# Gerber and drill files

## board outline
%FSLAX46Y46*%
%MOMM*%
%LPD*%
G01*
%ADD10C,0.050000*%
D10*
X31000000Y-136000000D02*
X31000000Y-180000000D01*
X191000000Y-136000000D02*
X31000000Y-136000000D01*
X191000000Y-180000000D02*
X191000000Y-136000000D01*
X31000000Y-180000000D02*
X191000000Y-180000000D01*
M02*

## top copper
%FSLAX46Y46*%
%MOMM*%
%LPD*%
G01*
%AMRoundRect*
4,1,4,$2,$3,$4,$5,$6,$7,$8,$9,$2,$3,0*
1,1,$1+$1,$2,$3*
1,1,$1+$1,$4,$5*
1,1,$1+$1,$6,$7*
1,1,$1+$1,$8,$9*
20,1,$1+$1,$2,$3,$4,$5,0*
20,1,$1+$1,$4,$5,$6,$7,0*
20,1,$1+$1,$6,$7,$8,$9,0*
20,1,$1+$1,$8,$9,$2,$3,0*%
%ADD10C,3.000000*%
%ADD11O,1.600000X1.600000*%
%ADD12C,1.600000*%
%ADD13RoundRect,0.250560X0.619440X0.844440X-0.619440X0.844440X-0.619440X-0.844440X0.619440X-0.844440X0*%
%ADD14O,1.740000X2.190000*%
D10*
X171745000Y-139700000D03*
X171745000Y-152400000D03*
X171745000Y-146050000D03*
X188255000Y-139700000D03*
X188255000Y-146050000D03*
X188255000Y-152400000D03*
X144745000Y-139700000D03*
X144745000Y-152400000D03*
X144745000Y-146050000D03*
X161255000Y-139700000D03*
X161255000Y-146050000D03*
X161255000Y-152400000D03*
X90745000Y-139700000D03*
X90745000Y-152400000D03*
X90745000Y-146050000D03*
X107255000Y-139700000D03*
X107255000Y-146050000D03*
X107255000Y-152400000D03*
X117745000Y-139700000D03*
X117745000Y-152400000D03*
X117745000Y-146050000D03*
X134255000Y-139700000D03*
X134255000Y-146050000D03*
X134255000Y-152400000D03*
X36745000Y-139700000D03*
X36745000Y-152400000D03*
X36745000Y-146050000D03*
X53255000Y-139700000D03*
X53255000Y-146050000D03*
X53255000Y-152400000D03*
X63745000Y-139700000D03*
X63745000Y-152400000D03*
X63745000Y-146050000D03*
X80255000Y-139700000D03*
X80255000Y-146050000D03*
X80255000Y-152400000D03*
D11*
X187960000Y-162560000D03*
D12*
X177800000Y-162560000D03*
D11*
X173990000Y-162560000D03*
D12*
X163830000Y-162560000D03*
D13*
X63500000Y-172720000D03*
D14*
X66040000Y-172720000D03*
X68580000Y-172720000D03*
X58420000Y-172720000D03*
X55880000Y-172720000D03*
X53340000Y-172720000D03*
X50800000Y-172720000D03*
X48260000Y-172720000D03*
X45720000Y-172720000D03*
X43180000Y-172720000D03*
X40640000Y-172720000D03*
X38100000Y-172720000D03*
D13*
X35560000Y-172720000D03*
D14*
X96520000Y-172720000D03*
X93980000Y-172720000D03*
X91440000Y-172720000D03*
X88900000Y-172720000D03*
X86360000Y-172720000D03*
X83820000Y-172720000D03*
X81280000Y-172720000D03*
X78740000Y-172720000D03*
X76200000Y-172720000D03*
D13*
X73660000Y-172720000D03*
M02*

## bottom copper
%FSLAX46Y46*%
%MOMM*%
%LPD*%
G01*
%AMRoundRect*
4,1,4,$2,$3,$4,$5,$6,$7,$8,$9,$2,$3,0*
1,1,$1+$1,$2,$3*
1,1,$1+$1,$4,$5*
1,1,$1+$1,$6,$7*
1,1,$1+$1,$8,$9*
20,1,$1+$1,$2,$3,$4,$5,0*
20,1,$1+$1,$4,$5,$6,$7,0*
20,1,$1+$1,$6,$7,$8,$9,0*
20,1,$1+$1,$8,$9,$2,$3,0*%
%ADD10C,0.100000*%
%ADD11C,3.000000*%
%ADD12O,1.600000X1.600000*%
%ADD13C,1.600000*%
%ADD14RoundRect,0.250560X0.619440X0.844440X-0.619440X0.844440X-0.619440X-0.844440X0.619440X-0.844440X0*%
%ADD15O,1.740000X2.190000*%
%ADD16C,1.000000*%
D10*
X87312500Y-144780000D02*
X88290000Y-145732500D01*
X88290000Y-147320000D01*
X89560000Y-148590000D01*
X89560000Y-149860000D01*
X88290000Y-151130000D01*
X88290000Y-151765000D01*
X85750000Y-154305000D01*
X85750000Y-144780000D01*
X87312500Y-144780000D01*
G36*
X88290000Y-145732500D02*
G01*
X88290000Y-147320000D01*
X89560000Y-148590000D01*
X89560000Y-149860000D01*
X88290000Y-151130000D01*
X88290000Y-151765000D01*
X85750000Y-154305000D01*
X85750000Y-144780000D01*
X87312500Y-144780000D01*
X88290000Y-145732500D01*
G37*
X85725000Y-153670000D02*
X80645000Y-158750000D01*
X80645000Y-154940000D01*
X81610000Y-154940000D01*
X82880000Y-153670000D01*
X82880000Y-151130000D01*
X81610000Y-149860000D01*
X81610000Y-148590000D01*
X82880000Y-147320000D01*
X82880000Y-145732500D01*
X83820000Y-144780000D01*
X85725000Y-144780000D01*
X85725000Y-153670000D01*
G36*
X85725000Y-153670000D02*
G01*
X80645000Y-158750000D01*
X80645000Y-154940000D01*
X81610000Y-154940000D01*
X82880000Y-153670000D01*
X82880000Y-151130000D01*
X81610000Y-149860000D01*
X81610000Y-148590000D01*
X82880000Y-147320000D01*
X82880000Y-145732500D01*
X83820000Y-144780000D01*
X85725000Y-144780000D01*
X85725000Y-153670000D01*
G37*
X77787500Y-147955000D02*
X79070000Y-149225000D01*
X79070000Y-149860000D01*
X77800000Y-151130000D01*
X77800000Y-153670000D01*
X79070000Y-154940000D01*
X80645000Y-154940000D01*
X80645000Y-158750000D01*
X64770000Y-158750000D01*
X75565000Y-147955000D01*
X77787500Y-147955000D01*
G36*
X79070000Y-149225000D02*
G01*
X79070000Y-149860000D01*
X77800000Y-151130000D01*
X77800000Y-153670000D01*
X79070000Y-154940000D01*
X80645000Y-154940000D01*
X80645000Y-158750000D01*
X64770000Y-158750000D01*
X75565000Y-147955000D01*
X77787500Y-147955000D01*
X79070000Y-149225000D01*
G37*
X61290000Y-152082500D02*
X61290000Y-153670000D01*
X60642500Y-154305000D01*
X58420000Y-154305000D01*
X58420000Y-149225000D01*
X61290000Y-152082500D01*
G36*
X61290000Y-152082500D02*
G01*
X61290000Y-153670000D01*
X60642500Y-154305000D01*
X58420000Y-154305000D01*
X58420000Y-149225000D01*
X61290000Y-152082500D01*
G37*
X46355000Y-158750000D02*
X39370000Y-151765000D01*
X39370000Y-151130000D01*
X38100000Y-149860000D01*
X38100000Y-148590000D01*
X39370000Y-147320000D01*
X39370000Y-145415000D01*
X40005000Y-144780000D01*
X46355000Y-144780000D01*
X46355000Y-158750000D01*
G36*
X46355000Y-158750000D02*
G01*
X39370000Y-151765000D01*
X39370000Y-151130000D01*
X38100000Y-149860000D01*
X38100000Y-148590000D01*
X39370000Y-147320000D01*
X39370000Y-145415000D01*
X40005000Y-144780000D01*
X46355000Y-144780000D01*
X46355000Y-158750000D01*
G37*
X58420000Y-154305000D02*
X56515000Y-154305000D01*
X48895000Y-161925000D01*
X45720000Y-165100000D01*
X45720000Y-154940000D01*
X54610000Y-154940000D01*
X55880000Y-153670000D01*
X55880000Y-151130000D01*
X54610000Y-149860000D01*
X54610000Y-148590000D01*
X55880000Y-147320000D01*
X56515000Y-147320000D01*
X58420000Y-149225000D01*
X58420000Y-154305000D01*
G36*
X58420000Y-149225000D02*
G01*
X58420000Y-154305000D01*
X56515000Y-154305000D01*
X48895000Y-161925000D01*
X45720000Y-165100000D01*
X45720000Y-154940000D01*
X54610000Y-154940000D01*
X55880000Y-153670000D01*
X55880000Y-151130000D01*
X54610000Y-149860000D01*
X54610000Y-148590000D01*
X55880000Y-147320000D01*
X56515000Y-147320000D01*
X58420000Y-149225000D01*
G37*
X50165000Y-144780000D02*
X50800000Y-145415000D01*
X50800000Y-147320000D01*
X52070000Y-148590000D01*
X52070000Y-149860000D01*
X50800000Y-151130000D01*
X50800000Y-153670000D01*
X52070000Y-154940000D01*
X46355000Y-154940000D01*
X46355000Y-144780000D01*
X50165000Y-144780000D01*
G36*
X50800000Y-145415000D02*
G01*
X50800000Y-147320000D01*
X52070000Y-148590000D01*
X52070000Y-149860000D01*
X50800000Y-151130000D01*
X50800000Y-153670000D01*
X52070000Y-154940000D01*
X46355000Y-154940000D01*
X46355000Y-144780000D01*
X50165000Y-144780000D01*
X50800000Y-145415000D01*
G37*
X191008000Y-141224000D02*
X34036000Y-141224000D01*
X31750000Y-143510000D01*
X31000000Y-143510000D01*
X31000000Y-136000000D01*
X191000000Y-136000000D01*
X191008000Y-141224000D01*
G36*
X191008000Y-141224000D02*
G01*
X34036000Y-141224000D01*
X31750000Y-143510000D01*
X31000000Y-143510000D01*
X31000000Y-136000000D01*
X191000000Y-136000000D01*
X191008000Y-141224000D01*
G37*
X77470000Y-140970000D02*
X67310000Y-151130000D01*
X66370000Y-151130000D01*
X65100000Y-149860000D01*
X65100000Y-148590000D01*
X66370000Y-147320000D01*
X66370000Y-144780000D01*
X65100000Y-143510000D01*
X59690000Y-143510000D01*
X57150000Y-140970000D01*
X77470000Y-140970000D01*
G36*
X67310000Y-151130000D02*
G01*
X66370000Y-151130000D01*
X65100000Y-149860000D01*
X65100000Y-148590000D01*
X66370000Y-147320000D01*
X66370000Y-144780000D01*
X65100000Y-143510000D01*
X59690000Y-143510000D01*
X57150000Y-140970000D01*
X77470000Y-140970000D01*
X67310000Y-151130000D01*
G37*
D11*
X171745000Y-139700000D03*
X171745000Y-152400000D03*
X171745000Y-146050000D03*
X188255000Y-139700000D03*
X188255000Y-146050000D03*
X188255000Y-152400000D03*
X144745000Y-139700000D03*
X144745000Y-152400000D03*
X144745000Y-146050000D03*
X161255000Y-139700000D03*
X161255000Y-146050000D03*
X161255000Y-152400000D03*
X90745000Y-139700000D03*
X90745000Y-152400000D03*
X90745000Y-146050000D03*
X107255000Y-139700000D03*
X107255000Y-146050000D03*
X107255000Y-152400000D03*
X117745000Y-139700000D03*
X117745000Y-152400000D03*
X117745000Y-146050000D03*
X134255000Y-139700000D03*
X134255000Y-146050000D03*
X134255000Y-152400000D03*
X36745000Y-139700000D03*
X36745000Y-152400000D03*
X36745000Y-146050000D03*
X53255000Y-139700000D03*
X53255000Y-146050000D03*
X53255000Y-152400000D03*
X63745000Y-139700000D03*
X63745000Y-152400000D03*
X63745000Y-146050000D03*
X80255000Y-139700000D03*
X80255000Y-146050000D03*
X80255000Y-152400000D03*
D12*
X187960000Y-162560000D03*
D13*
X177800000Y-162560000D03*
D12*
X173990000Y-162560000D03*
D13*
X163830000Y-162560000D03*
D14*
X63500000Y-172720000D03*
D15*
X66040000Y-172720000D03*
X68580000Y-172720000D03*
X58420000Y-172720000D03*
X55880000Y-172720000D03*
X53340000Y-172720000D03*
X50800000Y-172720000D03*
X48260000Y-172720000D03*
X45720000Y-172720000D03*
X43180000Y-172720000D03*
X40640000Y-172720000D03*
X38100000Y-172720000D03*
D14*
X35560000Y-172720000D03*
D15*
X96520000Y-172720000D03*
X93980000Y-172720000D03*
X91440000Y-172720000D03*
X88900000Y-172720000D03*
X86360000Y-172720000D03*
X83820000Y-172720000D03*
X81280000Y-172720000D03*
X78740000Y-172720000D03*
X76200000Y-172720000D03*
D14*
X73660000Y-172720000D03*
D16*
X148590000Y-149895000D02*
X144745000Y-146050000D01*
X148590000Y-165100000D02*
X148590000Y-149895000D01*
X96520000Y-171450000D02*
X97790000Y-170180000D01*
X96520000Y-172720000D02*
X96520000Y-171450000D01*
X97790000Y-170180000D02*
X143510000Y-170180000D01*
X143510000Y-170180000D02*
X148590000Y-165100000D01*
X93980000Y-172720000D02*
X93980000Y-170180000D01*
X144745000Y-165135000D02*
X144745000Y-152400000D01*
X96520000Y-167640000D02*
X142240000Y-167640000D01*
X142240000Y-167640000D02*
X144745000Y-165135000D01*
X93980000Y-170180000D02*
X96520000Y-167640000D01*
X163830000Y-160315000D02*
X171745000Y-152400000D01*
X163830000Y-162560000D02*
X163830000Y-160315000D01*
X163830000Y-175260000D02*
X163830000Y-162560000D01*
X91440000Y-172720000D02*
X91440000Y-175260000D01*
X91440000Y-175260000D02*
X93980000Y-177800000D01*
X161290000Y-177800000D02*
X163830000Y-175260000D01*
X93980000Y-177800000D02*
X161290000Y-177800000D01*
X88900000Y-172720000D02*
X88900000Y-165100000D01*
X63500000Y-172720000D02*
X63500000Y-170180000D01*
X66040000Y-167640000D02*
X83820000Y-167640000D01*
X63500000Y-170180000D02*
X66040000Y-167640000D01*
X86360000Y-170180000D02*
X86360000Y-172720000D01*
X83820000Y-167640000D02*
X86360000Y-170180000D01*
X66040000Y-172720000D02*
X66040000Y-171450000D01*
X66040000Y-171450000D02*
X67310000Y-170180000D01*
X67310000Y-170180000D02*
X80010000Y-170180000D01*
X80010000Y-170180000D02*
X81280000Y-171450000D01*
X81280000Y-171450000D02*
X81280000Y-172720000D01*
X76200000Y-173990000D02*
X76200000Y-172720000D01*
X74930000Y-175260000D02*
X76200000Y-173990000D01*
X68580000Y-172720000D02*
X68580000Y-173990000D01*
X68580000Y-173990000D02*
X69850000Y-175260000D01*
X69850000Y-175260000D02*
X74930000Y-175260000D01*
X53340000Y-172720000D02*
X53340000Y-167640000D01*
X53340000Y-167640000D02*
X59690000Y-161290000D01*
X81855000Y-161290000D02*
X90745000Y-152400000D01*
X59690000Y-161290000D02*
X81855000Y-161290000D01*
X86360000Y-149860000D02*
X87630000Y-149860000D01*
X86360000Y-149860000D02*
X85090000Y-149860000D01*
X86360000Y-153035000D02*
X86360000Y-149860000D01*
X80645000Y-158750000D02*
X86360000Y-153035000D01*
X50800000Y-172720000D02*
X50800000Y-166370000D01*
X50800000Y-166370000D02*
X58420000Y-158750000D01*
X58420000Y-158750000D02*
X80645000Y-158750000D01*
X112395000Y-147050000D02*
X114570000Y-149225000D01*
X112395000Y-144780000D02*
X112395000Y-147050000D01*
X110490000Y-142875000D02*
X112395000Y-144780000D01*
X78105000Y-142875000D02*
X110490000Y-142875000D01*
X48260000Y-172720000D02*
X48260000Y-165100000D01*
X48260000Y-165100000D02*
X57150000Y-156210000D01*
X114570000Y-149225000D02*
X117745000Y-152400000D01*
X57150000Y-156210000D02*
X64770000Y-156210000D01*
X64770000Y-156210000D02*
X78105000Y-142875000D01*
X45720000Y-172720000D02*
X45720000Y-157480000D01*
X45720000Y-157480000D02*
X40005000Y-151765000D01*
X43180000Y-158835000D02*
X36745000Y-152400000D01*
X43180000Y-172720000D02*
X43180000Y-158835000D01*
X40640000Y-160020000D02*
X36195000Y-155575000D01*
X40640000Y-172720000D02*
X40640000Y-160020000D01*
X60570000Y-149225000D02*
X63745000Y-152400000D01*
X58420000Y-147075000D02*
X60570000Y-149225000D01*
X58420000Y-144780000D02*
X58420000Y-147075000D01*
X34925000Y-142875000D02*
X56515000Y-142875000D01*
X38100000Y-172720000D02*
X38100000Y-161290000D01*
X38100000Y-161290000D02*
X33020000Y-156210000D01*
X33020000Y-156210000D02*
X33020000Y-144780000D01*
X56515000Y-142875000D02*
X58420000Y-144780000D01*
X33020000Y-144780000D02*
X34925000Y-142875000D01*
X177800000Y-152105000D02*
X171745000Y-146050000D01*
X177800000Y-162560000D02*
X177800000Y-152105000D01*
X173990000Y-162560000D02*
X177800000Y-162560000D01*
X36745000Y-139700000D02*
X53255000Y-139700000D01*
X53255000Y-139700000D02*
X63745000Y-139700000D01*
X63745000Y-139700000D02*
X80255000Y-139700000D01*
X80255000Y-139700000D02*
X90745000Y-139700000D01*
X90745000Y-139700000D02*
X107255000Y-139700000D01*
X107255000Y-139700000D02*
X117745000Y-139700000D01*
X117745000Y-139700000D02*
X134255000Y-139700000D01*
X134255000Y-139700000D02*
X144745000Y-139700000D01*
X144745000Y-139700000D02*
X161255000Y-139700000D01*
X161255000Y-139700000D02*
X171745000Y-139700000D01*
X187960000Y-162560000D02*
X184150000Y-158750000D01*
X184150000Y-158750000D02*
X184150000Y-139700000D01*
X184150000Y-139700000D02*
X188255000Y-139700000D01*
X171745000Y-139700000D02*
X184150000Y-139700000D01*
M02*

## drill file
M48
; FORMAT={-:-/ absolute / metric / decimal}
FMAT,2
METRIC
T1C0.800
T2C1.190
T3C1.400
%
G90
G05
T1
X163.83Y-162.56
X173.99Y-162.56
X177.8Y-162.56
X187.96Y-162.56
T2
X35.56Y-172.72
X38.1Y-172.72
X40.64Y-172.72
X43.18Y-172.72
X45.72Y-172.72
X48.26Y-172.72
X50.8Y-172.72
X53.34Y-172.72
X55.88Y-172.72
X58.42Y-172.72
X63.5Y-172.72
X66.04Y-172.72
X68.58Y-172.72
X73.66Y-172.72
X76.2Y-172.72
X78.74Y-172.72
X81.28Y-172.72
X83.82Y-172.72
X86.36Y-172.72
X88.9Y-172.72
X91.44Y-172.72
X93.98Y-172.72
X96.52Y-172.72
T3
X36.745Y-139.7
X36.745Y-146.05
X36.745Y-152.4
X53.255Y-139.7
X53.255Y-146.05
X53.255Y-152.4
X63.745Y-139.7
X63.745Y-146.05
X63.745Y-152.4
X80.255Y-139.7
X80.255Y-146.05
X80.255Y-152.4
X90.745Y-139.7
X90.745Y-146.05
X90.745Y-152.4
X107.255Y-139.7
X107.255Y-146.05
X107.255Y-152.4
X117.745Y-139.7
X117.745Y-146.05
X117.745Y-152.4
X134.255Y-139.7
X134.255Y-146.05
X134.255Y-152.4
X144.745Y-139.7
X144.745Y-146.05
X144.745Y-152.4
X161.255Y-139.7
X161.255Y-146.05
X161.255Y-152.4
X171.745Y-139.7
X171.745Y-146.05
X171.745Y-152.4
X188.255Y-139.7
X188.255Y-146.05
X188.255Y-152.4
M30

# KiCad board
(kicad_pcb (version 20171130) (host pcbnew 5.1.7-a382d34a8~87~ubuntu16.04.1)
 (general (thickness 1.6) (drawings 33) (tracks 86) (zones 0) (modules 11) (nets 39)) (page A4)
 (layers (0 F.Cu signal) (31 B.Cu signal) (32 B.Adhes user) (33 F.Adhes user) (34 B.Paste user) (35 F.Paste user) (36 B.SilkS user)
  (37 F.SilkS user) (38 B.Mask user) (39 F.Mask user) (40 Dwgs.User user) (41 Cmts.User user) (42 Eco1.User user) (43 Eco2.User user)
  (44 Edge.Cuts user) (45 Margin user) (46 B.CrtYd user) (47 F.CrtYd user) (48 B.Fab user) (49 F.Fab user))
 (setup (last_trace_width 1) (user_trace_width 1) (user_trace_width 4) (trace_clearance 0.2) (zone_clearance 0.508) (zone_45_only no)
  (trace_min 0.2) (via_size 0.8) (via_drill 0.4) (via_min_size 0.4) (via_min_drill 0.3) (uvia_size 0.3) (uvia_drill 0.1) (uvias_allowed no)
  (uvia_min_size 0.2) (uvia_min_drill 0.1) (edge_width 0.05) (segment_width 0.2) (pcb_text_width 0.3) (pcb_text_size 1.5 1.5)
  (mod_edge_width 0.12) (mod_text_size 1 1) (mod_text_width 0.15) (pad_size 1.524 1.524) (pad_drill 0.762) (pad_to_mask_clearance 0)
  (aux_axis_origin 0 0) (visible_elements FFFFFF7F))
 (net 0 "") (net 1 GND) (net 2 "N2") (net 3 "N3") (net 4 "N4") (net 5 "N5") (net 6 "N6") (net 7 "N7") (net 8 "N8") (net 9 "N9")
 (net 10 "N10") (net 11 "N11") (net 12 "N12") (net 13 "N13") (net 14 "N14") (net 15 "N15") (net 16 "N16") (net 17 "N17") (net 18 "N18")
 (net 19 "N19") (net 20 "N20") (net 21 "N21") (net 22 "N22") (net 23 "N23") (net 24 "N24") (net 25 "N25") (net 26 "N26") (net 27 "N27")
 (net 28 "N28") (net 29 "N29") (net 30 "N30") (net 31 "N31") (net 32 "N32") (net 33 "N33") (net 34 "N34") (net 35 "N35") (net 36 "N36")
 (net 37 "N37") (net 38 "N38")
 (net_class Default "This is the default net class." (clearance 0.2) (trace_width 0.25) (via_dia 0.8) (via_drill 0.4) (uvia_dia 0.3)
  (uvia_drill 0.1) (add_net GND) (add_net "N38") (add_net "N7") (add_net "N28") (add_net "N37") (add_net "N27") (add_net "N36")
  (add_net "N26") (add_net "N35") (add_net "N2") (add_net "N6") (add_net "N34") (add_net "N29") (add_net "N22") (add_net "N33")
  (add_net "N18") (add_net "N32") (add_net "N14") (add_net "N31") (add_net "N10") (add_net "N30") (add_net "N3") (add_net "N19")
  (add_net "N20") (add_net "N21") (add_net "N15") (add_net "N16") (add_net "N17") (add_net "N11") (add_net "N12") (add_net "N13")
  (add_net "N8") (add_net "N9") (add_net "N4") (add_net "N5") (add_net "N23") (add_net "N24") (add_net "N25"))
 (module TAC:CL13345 (layer F.Cu) (at 180 139.7 90)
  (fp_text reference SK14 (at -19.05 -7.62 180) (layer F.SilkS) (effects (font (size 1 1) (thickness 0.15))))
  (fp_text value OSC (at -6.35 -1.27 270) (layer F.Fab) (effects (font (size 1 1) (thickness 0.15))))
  (pad S thru_hole circle (at 0 -8.255 180) (size 3 3) (drill 1.4) (layers *.Cu *.Mask) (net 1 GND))
  (pad T thru_hole circle (at -12.7 -8.255 180) (size 3 3) (drill 1.4) (layers *.Cu *.Mask) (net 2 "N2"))
  (pad R thru_hole circle (at -6.35 -8.255 180) (size 3 3) (drill 1.4) (layers *.Cu *.Mask) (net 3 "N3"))
  (pad SN thru_hole circle (at 0 8.255 180) (size 3 3) (drill 1.4) (layers *.Cu *.Mask) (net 1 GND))
  (pad RN thru_hole circle (at -6.35 8.255 180) (size 3 3) (drill 1.4) (layers *.Cu *.Mask) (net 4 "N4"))
  (pad TN thru_hole circle (at -12.7 8.255 180) (size 3 3) (drill 1.4) (layers *.Cu *.Mask) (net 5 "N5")))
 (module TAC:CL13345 (layer F.Cu) (at 153 139.7 90)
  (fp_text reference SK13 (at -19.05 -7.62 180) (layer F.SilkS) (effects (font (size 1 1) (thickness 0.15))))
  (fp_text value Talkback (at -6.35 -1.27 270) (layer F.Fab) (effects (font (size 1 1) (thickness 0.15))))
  (pad S thru_hole circle (at 0 -8.255 180) (size 3 3) (drill 1.4) (layers *.Cu *.Mask) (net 1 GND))
  (pad T thru_hole circle (at -12.7 -8.255 180) (size 3 3) (drill 1.4) (layers *.Cu *.Mask) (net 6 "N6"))
  (pad R thru_hole circle (at -6.35 -8.255 180) (size 3 3) (drill 1.4) (layers *.Cu *.Mask) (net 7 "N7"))
  (pad SN thru_hole circle (at 0 8.255 180) (size 3 3) (drill 1.4) (layers *.Cu *.Mask) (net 1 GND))
  (pad RN thru_hole circle (at -6.35 8.255 180) (size 3 3) (drill 1.4) (layers *.Cu *.Mask) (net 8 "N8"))
  (pad TN thru_hole circle (at -12.7 8.255 180) (size 3 3) (drill 1.4) (layers *.Cu *.Mask) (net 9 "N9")))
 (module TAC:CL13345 (layer F.Cu) (at 99 139.7 90)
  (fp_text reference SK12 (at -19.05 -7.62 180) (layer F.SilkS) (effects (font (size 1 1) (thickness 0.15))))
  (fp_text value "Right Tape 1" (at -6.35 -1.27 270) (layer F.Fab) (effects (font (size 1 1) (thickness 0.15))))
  (pad S thru_hole circle (at 0 -8.255 180) (size 3 3) (drill 1.4) (layers *.Cu *.Mask) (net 1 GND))
  (pad T thru_hole circle (at -12.7 -8.255 180) (size 3 3) (drill 1.4) (layers *.Cu *.Mask) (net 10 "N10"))
  (pad R thru_hole circle (at -6.35 -8.255 180) (size 3 3) (drill 1.4) (layers *.Cu *.Mask) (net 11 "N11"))
  (pad SN thru_hole circle (at 0 8.255 180) (size 3 3) (drill 1.4) (layers *.Cu *.Mask) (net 1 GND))
  (pad RN thru_hole circle (at -6.35 8.255 180) (size 3 3) (drill 1.4) (layers *.Cu *.Mask) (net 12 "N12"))
  (pad TN thru_hole circle (at -12.7 8.255 180) (size 3 3) (drill 1.4) (layers *.Cu *.Mask) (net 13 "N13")))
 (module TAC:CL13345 (layer F.Cu) (at 126 139.7 90)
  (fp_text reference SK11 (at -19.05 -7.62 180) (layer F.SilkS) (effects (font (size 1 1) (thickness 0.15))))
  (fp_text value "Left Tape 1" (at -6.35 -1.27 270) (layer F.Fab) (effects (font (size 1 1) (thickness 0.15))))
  (pad S thru_hole circle (at 0 -8.255 180) (size 3 3) (drill 1.4) (layers *.Cu *.Mask) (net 1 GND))
  (pad T thru_hole circle (at -12.7 -8.255 180) (size 3 3) (drill 1.4) (layers *.Cu *.Mask) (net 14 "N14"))
  (pad R thru_hole circle (at -6.35 -8.255 180) (size 3 3) (drill 1.4) (layers *.Cu *.Mask) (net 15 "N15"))
  (pad SN thru_hole circle (at 0 8.255 180) (size 3 3) (drill 1.4) (layers *.Cu *.Mask) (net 1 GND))
  (pad RN thru_hole circle (at -6.35 8.255 180) (size 3 3) (drill 1.4) (layers *.Cu *.Mask) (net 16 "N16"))
  (pad TN thru_hole circle (at -12.7 8.255 180) (size 3 3) (drill 1.4) (layers *.Cu *.Mask) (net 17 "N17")))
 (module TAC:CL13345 (layer F.Cu) (at 45 139.7 90)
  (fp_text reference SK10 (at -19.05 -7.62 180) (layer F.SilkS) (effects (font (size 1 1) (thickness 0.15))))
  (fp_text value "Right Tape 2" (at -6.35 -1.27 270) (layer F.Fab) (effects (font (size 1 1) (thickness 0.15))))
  (pad S thru_hole circle (at 0 -8.255 180) (size 3 3) (drill 1.4) (layers *.Cu *.Mask) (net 1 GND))
  (pad T thru_hole circle (at -12.7 -8.255 180) (size 3 3) (drill 1.4) (layers *.Cu *.Mask) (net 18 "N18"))
  (pad R thru_hole circle (at -6.35 -8.255 180) (size 3 3) (drill 1.4) (layers *.Cu *.Mask) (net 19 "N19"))
  (pad SN thru_hole circle (at 0 8.255 180) (size 3 3) (drill 1.4) (layers *.Cu *.Mask) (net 1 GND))
  (pad RN thru_hole circle (at -6.35 8.255 180) (size 3 3) (drill 1.4) (layers *.Cu *.Mask) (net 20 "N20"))
  (pad TN thru_hole circle (at -12.7 8.255 180) (size 3 3) (drill 1.4) (layers *.Cu *.Mask) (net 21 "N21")))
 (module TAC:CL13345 (layer F.Cu) (at 72 139.7 90)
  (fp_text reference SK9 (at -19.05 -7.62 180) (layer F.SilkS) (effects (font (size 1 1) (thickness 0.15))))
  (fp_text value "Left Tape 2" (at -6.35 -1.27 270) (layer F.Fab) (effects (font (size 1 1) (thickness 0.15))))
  (pad S thru_hole circle (at 0 -8.255 180) (size 3 3) (drill 1.4) (layers *.Cu *.Mask) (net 1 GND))
  (pad T thru_hole circle (at -12.7 -8.255 180) (size 3 3) (drill 1.4) (layers *.Cu *.Mask) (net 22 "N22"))
  (pad R thru_hole circle (at -6.35 -8.255 180) (size 3 3) (drill 1.4) (layers *.Cu *.Mask) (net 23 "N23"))
  (pad SN thru_hole circle (at 0 8.255 180) (size 3 3) (drill 1.4) (layers *.Cu *.Mask) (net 1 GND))
  (pad RN thru_hole circle (at -6.35 8.255 180) (size 3 3) (drill 1.4) (layers *.Cu *.Mask) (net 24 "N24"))
  (pad TN thru_hole circle (at -12.7 8.255 180) (size 3 3) (drill 1.4) (layers *.Cu *.Mask) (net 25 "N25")))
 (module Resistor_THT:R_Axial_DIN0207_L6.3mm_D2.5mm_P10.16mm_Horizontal (layer F.Cu) (at 177.8 162.56)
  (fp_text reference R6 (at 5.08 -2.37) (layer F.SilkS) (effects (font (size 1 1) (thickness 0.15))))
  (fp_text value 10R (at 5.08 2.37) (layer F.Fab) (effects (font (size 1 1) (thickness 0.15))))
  (pad 2 thru_hole oval (at 10.16 0) (size 1.6 1.6) (drill 0.8) (layers *.Cu *.Mask) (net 1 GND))
  (pad 1 thru_hole circle (at 0 0) (size 1.6 1.6) (drill 0.8) (layers *.Cu *.Mask) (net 3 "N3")))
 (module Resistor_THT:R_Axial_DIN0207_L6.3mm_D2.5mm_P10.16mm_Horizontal (layer F.Cu) (at 163.83 162.56)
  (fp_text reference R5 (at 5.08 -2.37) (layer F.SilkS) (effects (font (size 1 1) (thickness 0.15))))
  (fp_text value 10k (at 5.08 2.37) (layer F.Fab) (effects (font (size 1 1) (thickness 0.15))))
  (pad 2 thru_hole oval (at 10.16 0) (size 1.6 1.6) (drill 0.8) (layers *.Cu *.Mask) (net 3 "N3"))
  (pad 1 thru_hole circle (at 0 0) (size 1.6 1.6) (drill 0.8) (layers *.Cu *.Mask) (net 2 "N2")))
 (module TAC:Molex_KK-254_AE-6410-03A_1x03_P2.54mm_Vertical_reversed (layer F.Cu) (at 68.58 172.72 180)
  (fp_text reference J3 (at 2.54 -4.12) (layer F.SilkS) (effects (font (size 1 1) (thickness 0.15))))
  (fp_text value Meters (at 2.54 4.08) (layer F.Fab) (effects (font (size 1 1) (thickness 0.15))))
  (pad 1 thru_hole roundrect (at 5.08 0 180) (size 1.74 2.19) (drill 1.19) (layers *.Cu *.Mask) (roundrect_rratio 0.144) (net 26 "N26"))
  (pad 2 thru_hole oval (at 2.54 0 180) (size 1.74 2.19) (drill 1.19) (layers *.Cu *.Mask) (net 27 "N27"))
  (pad 3 thru_hole oval (at 0 0 180) (size 1.74 2.19) (drill 1.19) (layers *.Cu *.Mask) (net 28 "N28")))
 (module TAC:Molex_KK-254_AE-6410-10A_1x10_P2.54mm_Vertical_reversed (layer F.Cu) (at 58.42 172.72 180)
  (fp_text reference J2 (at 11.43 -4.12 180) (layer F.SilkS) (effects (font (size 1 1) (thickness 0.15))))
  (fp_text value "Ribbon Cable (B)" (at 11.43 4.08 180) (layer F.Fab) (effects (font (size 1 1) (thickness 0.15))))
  (pad 10 thru_hole oval (at 0 0 180) (size 1.74 2.19) (drill 1.19) (layers *.Cu *.Mask) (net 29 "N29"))
  (pad 9 thru_hole oval (at 2.54 0 180) (size 1.74 2.19) (drill 1.19) (layers *.Cu *.Mask) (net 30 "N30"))
  (pad 8 thru_hole oval (at 5.08 0 180) (size 1.74 2.19) (drill 1.19) (layers *.Cu *.Mask) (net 10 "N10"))
  (pad 7 thru_hole oval (at 7.62 0 180) (size 1.74 2.19) (drill 1.19) (layers *.Cu *.Mask) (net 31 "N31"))
  (pad 6 thru_hole oval (at 10.16 0 180) (size 1.74 2.19) (drill 1.19) (layers *.Cu *.Mask) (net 14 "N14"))
  (pad 5 thru_hole oval (at 12.7 0 180) (size 1.74 2.19) (drill 1.19) (layers *.Cu *.Mask) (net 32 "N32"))
  (pad 4 thru_hole oval (at 15.24 0 180) (size 1.74 2.19) (drill 1.19) (layers *.Cu *.Mask) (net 18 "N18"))
  (pad 3 thru_hole oval (at 17.78 0 180) (size 1.74 2.19) (drill 1.19) (layers *.Cu *.Mask) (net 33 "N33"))
  (pad 2 thru_hole oval (at 20.32 0 180) (size 1.74 2.19) (drill 1.19) (layers *.Cu *.Mask) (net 22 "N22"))
  (pad 1 thru_hole roundrect (at 22.86 0 180) (size 1.74 2.19) (drill 1.19) (layers *.Cu *.Mask) (roundrect_rratio 0.144) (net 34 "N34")))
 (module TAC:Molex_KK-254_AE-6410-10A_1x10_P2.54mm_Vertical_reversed (layer F.Cu) (at 96.52 172.72 180)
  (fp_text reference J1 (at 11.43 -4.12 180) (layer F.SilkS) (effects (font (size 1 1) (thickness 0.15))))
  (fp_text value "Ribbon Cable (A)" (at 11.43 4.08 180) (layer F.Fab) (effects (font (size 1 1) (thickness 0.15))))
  (pad 10 thru_hole oval (at 0 0 180) (size 1.74 2.19) (drill 1.19) (layers *.Cu *.Mask) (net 7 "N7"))
  (pad 9 thru_hole oval (at 2.54 0 180) (size 1.74 2.19) (drill 1.19) (layers *.Cu *.Mask) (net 6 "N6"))
  (pad 8 thru_hole oval (at 5.08 0 180) (size 1.74 2.19) (drill 1.19) (layers *.Cu *.Mask) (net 2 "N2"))
  (pad 7 thru_hole oval (at 7.62 0 180) (size 1.74 2.19) (drill 1.19) (layers *.Cu *.Mask) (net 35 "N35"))
  (pad 6 thru_hole oval (at 10.16 0 180) (size 1.74 2.19) (drill 1.19) (layers *.Cu *.Mask) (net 26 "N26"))
  (pad 5 thru_hole oval (at 12.7 0 180) (size 1.74 2.19) (drill 1.19) (layers *.Cu *.Mask) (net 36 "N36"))
  (pad 4 thru_hole oval (at 15.24 0 180) (size 1.74 2.19) (drill 1.19) (layers *.Cu *.Mask) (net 27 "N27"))
  (pad 3 thru_hole oval (at 17.78 0 180) (size 1.74 2.19) (drill 1.19) (layers *.Cu *.Mask) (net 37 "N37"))
  (pad 2 thru_hole oval (at 20.32 0 180) (size 1.74 2.19) (drill 1.19) (layers *.Cu *.Mask) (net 28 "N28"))
  (pad 1 thru_hole roundrect (at 22.86 0 180) (size 1.74 2.19) (drill 1.19) (layers *.Cu *.Mask) (roundrect_rratio 0.144) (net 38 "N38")))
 (gr_poly
  (pts (xy 87.3125 144.78) (xy 88.29 145.7325) (xy 88.29 147.32) (xy 89.56 148.59) (xy 89.56 149.86) (xy 88.29 151.13) (xy 88.29 151.765)
   (xy 85.75 154.305) (xy 85.75 144.78))
  (layer B.Cu) (width 0.1))
 (gr_poly
  (pts (xy 85.725 153.67) (xy 80.645 158.75) (xy 80.645 154.94) (xy 81.61 154.94) (xy 82.88 153.67) (xy 82.88 151.13) (xy 81.61 149.86)
   (xy 81.61 148.59) (xy 82.88 147.32) (xy 82.88 145.7325) (xy 83.82 144.78) (xy 85.725 144.78))
  (layer B.Cu) (width 0.1))
 (gr_poly
  (pts (xy 77.7875 147.955) (xy 79.07 149.225) (xy 79.07 149.86) (xy 77.8 151.13) (xy 77.8 153.67) (xy 79.07 154.94) (xy 80.645 154.94)
   (xy 80.645 158.75) (xy 64.77 158.75) (xy 75.565 147.955))
  (layer B.Cu) (width 0.1))
 (gr_poly (pts (xy 61.29 152.0825) (xy 61.29 153.67) (xy 60.6425 154.305) (xy 58.42 154.305) (xy 58.42 149.225)) (layer B.Cu) (width 0.1))
 (gr_poly
  (pts (xy 46.355 158.75) (xy 39.37 151.765) (xy 39.37 151.13) (xy 38.1 149.86) (xy 38.1 148.59) (xy 39.37 147.32) (xy 39.37 145.415)
   (xy 40.005 144.78) (xy 46.355 144.78))
  (layer B.Cu) (width 0.1))
 (gr_poly
  (pts (xy 58.42 154.305) (xy 56.515 154.305) (xy 48.895 161.925) (xy 45.72 165.1) (xy 45.72 154.94) (xy 54.61 154.94) (xy 55.88 153.67)
   (xy 55.88 151.13) (xy 54.61 149.86) (xy 54.61 148.59) (xy 55.88 147.32) (xy 56.515 147.32) (xy 58.42 149.225))
  (layer B.Cu) (width 0.1))
 (gr_poly
  (pts (xy 50.165 144.78) (xy 50.8 145.415) (xy 50.8 147.32) (xy 52.07 148.59) (xy 52.07 149.86) (xy 50.8 151.13) (xy 50.8 153.67)
   (xy 52.07 154.94) (xy 46.355 154.94) (xy 46.355 144.78))
  (layer B.Cu) (width 0.1))
 (gr_poly (pts (xy 191.008 141.224) (xy 34.036 141.224) (xy 31.75 143.51) (xy 31 143.51) (xy 31 136) (xy 191 136)) (layer B.Cu) (width 0.1))
 (gr_poly
  (pts (xy 77.47 140.97) (xy 67.31 151.13) (xy 66.37 151.13) (xy 65.1 149.86) (xy 65.1 148.59) (xy 66.37 147.32) (xy 66.37 144.78)
   (xy 65.1 143.51) (xy 59.69 143.51) (xy 57.15 140.97))
  (layer B.Cu) (width 0.1))
 (gr_line (start 31 136) (end 31 180) (layer Edge.Cuts) (width 0.05))
 (gr_line (start 191 136) (end 31 136) (layer Edge.Cuts) (width 0.05))
 (gr_line (start 191 180) (end 191 136) (layer Edge.Cuts) (width 0.05))
 (gr_line (start 31 180) (end 191 180) (layer Edge.Cuts) (width 0.05))
 (segment (start 148.59 149.895) (end 144.745 146.05) (width 1) (layer B.Cu) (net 7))
 (segment (start 148.59 165.1) (end 148.59 149.895) (width 1) (layer B.Cu) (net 7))
 (segment (start 96.52 171.45) (end 97.79 170.18) (width 1) (layer B.Cu) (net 7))
 (segment (start 96.52 172.72) (end 96.52 171.45) (width 1) (layer B.Cu) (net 7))
 (segment (start 97.79 170.18) (end 143.51 170.18) (width 1) (layer B.Cu) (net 7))
 (segment (start 143.51 170.18) (end 148.59 165.1) (width 1) (layer B.Cu) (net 7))
 (segment (start 93.98 172.72) (end 93.98 170.18) (width 1) (layer B.Cu) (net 6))
 (segment (start 144.745 165.135) (end 144.745 152.4) (width 1) (layer B.Cu) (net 6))
 (segment (start 96.52 167.64) (end 142.24 167.64) (width 1) (layer B.Cu) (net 6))
 (segment (start 142.24 167.64) (end 144.745 165.135) (width 1) (layer B.Cu) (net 6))
 (segment (start 93.98 170.18) (end 96.52 167.64) (width 1) (layer B.Cu) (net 6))
 (segment (start 163.83 160.315) (end 171.745 152.4) (width 1) (layer B.Cu) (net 2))
 (segment (start 163.83 162.56) (end 163.83 160.315) (width 1) (layer B.Cu) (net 2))
 (segment (start 163.83 175.26) (end 163.83 162.56) (width 1) (layer B.Cu) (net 2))
 (segment (start 91.44 172.72) (end 91.44 175.26) (width 1) (layer B.Cu) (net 2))
 (segment (start 91.44 175.26) (end 93.98 177.8) (width 1) (layer B.Cu) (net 2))
 (segment (start 161.29 177.8) (end 163.83 175.26) (width 1) (layer B.Cu) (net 2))
 (segment (start 93.98 177.8) (end 161.29 177.8) (width 1) (layer B.Cu) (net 2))
 (segment (start 88.9 172.72) (end 88.9 165.1) (width 1) (layer B.Cu) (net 35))
 (segment (start 63.5 172.72) (end 63.5 170.18) (width 1) (layer B.Cu) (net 26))
 (segment (start 66.04 167.64) (end 83.82 167.64) (width 1) (layer B.Cu) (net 26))
 (segment (start 63.5 170.18) (end 66.04 167.64) (width 1) (layer B.Cu) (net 26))
 (segment (start 86.36 170.18) (end 86.36 172.72) (width 1) (layer B.Cu) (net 26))
 (segment (start 83.82 167.64) (end 86.36 170.18) (width 1) (layer B.Cu) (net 26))
 (segment (start 66.04 172.72) (end 66.04 171.45) (width 1) (layer B.Cu) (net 27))
 (segment (start 66.04 171.45) (end 67.31 170.18) (width 1) (layer B.Cu) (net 27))
 (segment (start 67.31 170.18) (end 80.01 170.18) (width 1) (layer B.Cu) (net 27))
 (segment (start 80.01 170.18) (end 81.28 171.45) (width 1) (layer B.Cu) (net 27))
 (segment (start 81.28 171.45) (end 81.28 172.72) (width 1) (layer B.Cu) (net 27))
 (segment (start 76.2 173.99) (end 76.2 172.72) (width 1) (layer B.Cu) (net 28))
 (segment (start 74.93 175.26) (end 76.2 173.99) (width 1) (layer B.Cu) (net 28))
 (segment (start 68.58 172.72) (end 68.58 173.99) (width 1) (layer B.Cu) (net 28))
 (segment (start 68.58 173.99) (end 69.85 175.26) (width 1) (layer B.Cu) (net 28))
 (segment (start 69.85 175.26) (end 74.93 175.26) (width 1) (layer B.Cu) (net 28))
 (segment (start 53.34 172.72) (end 53.34 167.64) (width 1) (layer B.Cu) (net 10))
 (segment (start 53.34 167.64) (end 59.69 161.29) (width 1) (layer B.Cu) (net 10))
 (segment (start 81.855 161.29) (end 90.745 152.4) (width 1) (layer B.Cu) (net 10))
 (segment (start 59.69 161.29) (end 81.855 161.29) (width 1) (layer B.Cu) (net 10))
 (segment (start 86.36 149.86) (end 87.63 149.86) (width 1) (layer B.Cu) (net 31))
 (segment (start 86.36 149.86) (end 85.09 149.86) (width 1) (layer B.Cu) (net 31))
 (segment (start 86.36 153.035) (end 86.36 149.86) (width 1) (layer B.Cu) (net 31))
 (segment (start 80.645 158.75) (end 86.36 153.035) (width 1) (layer B.Cu) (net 31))
 (segment (start 50.8 172.72) (end 50.8 166.37) (width 1) (layer B.Cu) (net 31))
 (segment (start 50.8 166.37) (end 58.42 158.75) (width 1) (layer B.Cu) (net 31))
 (segment (start 58.42 158.75) (end 80.645 158.75) (width 1) (layer B.Cu) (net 31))
 (segment (start 112.395 147.05) (end 114.57 149.225) (width 1) (layer B.Cu) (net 14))
 (segment (start 112.395 144.78) (end 112.395 147.05) (width 1) (layer B.Cu) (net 14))
 (segment (start 110.49 142.875) (end 112.395 144.78) (width 1) (layer B.Cu) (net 14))
 (segment (start 78.105 142.875) (end 110.49 142.875) (width 1) (layer B.Cu) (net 14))
 (segment (start 48.26 172.72) (end 48.26 165.1) (width 1) (layer B.Cu) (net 14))
 (segment (start 48.26 165.1) (end 57.15 156.21) (width 1) (layer B.Cu) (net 14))
 (segment (start 114.57 149.225) (end 117.745 152.4) (width 1) (layer B.Cu) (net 14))
 (segment (start 57.15 156.21) (end 64.77 156.21) (width 1) (layer B.Cu) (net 14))
 (segment (start 64.77 156.21) (end 78.105 142.875) (width 1) (layer B.Cu) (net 14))
 (segment (start 45.72 172.72) (end 45.72 157.48) (width 1) (layer B.Cu) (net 32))
 (segment (start 45.72 157.48) (end 40.005 151.765) (width 1) (layer B.Cu) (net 32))
 (segment (start 43.18 158.835) (end 36.745 152.4) (width 1) (layer B.Cu) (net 18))
 (segment (start 43.18 172.72) (end 43.18 158.835) (width 1) (layer B.Cu) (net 18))
 (segment (start 40.64 160.02) (end 36.195 155.575) (width 1) (layer B.Cu) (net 33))
 (segment (start 40.64 172.72) (end 40.64 160.02) (width 1) (layer B.Cu) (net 33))
 (segment (start 60.57 149.225) (end 63.745 152.4) (width 1) (layer B.Cu) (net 22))
 (segment (start 58.42 147.075) (end 60.57 149.225) (width 1) (layer B.Cu) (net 22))
 (segment (start 58.42 144.78) (end 58.42 147.075) (width 1) (layer B.Cu) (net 22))
 (segment (start 34.925 142.875) (end 56.515 142.875) (width 1) (layer B.Cu) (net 22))
 (segment (start 38.1 172.72) (end 38.1 161.29) (width 1) (layer B.Cu) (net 22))
 (segment (start 38.1 161.29) (end 33.02 156.21) (width 1) (layer B.Cu) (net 22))
 (segment (start 33.02 156.21) (end 33.02 144.78) (width 1) (layer B.Cu) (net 22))
 (segment (start 56.515 142.875) (end 58.42 144.78) (width 1) (layer B.Cu) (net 22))
 (segment (start 33.02 144.78) (end 34.925 142.875) (width 1) (layer B.Cu) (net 22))
 (segment (start 177.8 152.105) (end 171.745 146.05) (width 1) (layer B.Cu) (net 3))
 (segment (start 177.8 162.56) (end 177.8 152.105) (width 1) (layer B.Cu) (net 3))
 (segment (start 173.99 162.56) (end 177.8 162.56) (width 1) (layer B.Cu) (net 3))
 (segment (start 36.745 139.7) (end 53.255 139.7) (width 1) (layer B.Cu) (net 1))
 (segment (start 53.255 139.7) (end 63.745 139.7) (width 1) (layer B.Cu) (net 1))
 (segment (start 63.745 139.7) (end 80.255 139.7) (width 1) (layer B.Cu) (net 1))
 (segment (start 80.255 139.7) (end 90.745 139.7) (width 1) (layer B.Cu) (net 1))
 (segment (start 90.745 139.7) (end 107.255 139.7) (width 1) (layer B.Cu) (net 1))
 (segment (start 107.255 139.7) (end 117.745 139.7) (width 1) (layer B.Cu) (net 1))
 (segment (start 117.745 139.7) (end 134.255 139.7) (width 1) (layer B.Cu) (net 1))
 (segment (start 134.255 139.7) (end 144.745 139.7) (width 1) (layer B.Cu) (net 1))
 (segment (start 144.745 139.7) (end 161.255 139.7) (width 1) (layer B.Cu) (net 1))
 (segment (start 161.255 139.7) (end 171.745 139.7) (width 1) (layer B.Cu) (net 1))
 (segment (start 187.96 162.56) (end 184.15 158.75) (width 1) (layer B.Cu) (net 1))
 (segment (start 184.15 158.75) (end 184.15 139.7) (width 1) (layer B.Cu) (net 1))
 (segment (start 184.15 139.7) (end 188.255 139.7) (width 1) (layer B.Cu) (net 1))
 (segment (start 171.745 139.7) (end 184.15 139.7) (width 1) (layer B.Cu) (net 1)))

